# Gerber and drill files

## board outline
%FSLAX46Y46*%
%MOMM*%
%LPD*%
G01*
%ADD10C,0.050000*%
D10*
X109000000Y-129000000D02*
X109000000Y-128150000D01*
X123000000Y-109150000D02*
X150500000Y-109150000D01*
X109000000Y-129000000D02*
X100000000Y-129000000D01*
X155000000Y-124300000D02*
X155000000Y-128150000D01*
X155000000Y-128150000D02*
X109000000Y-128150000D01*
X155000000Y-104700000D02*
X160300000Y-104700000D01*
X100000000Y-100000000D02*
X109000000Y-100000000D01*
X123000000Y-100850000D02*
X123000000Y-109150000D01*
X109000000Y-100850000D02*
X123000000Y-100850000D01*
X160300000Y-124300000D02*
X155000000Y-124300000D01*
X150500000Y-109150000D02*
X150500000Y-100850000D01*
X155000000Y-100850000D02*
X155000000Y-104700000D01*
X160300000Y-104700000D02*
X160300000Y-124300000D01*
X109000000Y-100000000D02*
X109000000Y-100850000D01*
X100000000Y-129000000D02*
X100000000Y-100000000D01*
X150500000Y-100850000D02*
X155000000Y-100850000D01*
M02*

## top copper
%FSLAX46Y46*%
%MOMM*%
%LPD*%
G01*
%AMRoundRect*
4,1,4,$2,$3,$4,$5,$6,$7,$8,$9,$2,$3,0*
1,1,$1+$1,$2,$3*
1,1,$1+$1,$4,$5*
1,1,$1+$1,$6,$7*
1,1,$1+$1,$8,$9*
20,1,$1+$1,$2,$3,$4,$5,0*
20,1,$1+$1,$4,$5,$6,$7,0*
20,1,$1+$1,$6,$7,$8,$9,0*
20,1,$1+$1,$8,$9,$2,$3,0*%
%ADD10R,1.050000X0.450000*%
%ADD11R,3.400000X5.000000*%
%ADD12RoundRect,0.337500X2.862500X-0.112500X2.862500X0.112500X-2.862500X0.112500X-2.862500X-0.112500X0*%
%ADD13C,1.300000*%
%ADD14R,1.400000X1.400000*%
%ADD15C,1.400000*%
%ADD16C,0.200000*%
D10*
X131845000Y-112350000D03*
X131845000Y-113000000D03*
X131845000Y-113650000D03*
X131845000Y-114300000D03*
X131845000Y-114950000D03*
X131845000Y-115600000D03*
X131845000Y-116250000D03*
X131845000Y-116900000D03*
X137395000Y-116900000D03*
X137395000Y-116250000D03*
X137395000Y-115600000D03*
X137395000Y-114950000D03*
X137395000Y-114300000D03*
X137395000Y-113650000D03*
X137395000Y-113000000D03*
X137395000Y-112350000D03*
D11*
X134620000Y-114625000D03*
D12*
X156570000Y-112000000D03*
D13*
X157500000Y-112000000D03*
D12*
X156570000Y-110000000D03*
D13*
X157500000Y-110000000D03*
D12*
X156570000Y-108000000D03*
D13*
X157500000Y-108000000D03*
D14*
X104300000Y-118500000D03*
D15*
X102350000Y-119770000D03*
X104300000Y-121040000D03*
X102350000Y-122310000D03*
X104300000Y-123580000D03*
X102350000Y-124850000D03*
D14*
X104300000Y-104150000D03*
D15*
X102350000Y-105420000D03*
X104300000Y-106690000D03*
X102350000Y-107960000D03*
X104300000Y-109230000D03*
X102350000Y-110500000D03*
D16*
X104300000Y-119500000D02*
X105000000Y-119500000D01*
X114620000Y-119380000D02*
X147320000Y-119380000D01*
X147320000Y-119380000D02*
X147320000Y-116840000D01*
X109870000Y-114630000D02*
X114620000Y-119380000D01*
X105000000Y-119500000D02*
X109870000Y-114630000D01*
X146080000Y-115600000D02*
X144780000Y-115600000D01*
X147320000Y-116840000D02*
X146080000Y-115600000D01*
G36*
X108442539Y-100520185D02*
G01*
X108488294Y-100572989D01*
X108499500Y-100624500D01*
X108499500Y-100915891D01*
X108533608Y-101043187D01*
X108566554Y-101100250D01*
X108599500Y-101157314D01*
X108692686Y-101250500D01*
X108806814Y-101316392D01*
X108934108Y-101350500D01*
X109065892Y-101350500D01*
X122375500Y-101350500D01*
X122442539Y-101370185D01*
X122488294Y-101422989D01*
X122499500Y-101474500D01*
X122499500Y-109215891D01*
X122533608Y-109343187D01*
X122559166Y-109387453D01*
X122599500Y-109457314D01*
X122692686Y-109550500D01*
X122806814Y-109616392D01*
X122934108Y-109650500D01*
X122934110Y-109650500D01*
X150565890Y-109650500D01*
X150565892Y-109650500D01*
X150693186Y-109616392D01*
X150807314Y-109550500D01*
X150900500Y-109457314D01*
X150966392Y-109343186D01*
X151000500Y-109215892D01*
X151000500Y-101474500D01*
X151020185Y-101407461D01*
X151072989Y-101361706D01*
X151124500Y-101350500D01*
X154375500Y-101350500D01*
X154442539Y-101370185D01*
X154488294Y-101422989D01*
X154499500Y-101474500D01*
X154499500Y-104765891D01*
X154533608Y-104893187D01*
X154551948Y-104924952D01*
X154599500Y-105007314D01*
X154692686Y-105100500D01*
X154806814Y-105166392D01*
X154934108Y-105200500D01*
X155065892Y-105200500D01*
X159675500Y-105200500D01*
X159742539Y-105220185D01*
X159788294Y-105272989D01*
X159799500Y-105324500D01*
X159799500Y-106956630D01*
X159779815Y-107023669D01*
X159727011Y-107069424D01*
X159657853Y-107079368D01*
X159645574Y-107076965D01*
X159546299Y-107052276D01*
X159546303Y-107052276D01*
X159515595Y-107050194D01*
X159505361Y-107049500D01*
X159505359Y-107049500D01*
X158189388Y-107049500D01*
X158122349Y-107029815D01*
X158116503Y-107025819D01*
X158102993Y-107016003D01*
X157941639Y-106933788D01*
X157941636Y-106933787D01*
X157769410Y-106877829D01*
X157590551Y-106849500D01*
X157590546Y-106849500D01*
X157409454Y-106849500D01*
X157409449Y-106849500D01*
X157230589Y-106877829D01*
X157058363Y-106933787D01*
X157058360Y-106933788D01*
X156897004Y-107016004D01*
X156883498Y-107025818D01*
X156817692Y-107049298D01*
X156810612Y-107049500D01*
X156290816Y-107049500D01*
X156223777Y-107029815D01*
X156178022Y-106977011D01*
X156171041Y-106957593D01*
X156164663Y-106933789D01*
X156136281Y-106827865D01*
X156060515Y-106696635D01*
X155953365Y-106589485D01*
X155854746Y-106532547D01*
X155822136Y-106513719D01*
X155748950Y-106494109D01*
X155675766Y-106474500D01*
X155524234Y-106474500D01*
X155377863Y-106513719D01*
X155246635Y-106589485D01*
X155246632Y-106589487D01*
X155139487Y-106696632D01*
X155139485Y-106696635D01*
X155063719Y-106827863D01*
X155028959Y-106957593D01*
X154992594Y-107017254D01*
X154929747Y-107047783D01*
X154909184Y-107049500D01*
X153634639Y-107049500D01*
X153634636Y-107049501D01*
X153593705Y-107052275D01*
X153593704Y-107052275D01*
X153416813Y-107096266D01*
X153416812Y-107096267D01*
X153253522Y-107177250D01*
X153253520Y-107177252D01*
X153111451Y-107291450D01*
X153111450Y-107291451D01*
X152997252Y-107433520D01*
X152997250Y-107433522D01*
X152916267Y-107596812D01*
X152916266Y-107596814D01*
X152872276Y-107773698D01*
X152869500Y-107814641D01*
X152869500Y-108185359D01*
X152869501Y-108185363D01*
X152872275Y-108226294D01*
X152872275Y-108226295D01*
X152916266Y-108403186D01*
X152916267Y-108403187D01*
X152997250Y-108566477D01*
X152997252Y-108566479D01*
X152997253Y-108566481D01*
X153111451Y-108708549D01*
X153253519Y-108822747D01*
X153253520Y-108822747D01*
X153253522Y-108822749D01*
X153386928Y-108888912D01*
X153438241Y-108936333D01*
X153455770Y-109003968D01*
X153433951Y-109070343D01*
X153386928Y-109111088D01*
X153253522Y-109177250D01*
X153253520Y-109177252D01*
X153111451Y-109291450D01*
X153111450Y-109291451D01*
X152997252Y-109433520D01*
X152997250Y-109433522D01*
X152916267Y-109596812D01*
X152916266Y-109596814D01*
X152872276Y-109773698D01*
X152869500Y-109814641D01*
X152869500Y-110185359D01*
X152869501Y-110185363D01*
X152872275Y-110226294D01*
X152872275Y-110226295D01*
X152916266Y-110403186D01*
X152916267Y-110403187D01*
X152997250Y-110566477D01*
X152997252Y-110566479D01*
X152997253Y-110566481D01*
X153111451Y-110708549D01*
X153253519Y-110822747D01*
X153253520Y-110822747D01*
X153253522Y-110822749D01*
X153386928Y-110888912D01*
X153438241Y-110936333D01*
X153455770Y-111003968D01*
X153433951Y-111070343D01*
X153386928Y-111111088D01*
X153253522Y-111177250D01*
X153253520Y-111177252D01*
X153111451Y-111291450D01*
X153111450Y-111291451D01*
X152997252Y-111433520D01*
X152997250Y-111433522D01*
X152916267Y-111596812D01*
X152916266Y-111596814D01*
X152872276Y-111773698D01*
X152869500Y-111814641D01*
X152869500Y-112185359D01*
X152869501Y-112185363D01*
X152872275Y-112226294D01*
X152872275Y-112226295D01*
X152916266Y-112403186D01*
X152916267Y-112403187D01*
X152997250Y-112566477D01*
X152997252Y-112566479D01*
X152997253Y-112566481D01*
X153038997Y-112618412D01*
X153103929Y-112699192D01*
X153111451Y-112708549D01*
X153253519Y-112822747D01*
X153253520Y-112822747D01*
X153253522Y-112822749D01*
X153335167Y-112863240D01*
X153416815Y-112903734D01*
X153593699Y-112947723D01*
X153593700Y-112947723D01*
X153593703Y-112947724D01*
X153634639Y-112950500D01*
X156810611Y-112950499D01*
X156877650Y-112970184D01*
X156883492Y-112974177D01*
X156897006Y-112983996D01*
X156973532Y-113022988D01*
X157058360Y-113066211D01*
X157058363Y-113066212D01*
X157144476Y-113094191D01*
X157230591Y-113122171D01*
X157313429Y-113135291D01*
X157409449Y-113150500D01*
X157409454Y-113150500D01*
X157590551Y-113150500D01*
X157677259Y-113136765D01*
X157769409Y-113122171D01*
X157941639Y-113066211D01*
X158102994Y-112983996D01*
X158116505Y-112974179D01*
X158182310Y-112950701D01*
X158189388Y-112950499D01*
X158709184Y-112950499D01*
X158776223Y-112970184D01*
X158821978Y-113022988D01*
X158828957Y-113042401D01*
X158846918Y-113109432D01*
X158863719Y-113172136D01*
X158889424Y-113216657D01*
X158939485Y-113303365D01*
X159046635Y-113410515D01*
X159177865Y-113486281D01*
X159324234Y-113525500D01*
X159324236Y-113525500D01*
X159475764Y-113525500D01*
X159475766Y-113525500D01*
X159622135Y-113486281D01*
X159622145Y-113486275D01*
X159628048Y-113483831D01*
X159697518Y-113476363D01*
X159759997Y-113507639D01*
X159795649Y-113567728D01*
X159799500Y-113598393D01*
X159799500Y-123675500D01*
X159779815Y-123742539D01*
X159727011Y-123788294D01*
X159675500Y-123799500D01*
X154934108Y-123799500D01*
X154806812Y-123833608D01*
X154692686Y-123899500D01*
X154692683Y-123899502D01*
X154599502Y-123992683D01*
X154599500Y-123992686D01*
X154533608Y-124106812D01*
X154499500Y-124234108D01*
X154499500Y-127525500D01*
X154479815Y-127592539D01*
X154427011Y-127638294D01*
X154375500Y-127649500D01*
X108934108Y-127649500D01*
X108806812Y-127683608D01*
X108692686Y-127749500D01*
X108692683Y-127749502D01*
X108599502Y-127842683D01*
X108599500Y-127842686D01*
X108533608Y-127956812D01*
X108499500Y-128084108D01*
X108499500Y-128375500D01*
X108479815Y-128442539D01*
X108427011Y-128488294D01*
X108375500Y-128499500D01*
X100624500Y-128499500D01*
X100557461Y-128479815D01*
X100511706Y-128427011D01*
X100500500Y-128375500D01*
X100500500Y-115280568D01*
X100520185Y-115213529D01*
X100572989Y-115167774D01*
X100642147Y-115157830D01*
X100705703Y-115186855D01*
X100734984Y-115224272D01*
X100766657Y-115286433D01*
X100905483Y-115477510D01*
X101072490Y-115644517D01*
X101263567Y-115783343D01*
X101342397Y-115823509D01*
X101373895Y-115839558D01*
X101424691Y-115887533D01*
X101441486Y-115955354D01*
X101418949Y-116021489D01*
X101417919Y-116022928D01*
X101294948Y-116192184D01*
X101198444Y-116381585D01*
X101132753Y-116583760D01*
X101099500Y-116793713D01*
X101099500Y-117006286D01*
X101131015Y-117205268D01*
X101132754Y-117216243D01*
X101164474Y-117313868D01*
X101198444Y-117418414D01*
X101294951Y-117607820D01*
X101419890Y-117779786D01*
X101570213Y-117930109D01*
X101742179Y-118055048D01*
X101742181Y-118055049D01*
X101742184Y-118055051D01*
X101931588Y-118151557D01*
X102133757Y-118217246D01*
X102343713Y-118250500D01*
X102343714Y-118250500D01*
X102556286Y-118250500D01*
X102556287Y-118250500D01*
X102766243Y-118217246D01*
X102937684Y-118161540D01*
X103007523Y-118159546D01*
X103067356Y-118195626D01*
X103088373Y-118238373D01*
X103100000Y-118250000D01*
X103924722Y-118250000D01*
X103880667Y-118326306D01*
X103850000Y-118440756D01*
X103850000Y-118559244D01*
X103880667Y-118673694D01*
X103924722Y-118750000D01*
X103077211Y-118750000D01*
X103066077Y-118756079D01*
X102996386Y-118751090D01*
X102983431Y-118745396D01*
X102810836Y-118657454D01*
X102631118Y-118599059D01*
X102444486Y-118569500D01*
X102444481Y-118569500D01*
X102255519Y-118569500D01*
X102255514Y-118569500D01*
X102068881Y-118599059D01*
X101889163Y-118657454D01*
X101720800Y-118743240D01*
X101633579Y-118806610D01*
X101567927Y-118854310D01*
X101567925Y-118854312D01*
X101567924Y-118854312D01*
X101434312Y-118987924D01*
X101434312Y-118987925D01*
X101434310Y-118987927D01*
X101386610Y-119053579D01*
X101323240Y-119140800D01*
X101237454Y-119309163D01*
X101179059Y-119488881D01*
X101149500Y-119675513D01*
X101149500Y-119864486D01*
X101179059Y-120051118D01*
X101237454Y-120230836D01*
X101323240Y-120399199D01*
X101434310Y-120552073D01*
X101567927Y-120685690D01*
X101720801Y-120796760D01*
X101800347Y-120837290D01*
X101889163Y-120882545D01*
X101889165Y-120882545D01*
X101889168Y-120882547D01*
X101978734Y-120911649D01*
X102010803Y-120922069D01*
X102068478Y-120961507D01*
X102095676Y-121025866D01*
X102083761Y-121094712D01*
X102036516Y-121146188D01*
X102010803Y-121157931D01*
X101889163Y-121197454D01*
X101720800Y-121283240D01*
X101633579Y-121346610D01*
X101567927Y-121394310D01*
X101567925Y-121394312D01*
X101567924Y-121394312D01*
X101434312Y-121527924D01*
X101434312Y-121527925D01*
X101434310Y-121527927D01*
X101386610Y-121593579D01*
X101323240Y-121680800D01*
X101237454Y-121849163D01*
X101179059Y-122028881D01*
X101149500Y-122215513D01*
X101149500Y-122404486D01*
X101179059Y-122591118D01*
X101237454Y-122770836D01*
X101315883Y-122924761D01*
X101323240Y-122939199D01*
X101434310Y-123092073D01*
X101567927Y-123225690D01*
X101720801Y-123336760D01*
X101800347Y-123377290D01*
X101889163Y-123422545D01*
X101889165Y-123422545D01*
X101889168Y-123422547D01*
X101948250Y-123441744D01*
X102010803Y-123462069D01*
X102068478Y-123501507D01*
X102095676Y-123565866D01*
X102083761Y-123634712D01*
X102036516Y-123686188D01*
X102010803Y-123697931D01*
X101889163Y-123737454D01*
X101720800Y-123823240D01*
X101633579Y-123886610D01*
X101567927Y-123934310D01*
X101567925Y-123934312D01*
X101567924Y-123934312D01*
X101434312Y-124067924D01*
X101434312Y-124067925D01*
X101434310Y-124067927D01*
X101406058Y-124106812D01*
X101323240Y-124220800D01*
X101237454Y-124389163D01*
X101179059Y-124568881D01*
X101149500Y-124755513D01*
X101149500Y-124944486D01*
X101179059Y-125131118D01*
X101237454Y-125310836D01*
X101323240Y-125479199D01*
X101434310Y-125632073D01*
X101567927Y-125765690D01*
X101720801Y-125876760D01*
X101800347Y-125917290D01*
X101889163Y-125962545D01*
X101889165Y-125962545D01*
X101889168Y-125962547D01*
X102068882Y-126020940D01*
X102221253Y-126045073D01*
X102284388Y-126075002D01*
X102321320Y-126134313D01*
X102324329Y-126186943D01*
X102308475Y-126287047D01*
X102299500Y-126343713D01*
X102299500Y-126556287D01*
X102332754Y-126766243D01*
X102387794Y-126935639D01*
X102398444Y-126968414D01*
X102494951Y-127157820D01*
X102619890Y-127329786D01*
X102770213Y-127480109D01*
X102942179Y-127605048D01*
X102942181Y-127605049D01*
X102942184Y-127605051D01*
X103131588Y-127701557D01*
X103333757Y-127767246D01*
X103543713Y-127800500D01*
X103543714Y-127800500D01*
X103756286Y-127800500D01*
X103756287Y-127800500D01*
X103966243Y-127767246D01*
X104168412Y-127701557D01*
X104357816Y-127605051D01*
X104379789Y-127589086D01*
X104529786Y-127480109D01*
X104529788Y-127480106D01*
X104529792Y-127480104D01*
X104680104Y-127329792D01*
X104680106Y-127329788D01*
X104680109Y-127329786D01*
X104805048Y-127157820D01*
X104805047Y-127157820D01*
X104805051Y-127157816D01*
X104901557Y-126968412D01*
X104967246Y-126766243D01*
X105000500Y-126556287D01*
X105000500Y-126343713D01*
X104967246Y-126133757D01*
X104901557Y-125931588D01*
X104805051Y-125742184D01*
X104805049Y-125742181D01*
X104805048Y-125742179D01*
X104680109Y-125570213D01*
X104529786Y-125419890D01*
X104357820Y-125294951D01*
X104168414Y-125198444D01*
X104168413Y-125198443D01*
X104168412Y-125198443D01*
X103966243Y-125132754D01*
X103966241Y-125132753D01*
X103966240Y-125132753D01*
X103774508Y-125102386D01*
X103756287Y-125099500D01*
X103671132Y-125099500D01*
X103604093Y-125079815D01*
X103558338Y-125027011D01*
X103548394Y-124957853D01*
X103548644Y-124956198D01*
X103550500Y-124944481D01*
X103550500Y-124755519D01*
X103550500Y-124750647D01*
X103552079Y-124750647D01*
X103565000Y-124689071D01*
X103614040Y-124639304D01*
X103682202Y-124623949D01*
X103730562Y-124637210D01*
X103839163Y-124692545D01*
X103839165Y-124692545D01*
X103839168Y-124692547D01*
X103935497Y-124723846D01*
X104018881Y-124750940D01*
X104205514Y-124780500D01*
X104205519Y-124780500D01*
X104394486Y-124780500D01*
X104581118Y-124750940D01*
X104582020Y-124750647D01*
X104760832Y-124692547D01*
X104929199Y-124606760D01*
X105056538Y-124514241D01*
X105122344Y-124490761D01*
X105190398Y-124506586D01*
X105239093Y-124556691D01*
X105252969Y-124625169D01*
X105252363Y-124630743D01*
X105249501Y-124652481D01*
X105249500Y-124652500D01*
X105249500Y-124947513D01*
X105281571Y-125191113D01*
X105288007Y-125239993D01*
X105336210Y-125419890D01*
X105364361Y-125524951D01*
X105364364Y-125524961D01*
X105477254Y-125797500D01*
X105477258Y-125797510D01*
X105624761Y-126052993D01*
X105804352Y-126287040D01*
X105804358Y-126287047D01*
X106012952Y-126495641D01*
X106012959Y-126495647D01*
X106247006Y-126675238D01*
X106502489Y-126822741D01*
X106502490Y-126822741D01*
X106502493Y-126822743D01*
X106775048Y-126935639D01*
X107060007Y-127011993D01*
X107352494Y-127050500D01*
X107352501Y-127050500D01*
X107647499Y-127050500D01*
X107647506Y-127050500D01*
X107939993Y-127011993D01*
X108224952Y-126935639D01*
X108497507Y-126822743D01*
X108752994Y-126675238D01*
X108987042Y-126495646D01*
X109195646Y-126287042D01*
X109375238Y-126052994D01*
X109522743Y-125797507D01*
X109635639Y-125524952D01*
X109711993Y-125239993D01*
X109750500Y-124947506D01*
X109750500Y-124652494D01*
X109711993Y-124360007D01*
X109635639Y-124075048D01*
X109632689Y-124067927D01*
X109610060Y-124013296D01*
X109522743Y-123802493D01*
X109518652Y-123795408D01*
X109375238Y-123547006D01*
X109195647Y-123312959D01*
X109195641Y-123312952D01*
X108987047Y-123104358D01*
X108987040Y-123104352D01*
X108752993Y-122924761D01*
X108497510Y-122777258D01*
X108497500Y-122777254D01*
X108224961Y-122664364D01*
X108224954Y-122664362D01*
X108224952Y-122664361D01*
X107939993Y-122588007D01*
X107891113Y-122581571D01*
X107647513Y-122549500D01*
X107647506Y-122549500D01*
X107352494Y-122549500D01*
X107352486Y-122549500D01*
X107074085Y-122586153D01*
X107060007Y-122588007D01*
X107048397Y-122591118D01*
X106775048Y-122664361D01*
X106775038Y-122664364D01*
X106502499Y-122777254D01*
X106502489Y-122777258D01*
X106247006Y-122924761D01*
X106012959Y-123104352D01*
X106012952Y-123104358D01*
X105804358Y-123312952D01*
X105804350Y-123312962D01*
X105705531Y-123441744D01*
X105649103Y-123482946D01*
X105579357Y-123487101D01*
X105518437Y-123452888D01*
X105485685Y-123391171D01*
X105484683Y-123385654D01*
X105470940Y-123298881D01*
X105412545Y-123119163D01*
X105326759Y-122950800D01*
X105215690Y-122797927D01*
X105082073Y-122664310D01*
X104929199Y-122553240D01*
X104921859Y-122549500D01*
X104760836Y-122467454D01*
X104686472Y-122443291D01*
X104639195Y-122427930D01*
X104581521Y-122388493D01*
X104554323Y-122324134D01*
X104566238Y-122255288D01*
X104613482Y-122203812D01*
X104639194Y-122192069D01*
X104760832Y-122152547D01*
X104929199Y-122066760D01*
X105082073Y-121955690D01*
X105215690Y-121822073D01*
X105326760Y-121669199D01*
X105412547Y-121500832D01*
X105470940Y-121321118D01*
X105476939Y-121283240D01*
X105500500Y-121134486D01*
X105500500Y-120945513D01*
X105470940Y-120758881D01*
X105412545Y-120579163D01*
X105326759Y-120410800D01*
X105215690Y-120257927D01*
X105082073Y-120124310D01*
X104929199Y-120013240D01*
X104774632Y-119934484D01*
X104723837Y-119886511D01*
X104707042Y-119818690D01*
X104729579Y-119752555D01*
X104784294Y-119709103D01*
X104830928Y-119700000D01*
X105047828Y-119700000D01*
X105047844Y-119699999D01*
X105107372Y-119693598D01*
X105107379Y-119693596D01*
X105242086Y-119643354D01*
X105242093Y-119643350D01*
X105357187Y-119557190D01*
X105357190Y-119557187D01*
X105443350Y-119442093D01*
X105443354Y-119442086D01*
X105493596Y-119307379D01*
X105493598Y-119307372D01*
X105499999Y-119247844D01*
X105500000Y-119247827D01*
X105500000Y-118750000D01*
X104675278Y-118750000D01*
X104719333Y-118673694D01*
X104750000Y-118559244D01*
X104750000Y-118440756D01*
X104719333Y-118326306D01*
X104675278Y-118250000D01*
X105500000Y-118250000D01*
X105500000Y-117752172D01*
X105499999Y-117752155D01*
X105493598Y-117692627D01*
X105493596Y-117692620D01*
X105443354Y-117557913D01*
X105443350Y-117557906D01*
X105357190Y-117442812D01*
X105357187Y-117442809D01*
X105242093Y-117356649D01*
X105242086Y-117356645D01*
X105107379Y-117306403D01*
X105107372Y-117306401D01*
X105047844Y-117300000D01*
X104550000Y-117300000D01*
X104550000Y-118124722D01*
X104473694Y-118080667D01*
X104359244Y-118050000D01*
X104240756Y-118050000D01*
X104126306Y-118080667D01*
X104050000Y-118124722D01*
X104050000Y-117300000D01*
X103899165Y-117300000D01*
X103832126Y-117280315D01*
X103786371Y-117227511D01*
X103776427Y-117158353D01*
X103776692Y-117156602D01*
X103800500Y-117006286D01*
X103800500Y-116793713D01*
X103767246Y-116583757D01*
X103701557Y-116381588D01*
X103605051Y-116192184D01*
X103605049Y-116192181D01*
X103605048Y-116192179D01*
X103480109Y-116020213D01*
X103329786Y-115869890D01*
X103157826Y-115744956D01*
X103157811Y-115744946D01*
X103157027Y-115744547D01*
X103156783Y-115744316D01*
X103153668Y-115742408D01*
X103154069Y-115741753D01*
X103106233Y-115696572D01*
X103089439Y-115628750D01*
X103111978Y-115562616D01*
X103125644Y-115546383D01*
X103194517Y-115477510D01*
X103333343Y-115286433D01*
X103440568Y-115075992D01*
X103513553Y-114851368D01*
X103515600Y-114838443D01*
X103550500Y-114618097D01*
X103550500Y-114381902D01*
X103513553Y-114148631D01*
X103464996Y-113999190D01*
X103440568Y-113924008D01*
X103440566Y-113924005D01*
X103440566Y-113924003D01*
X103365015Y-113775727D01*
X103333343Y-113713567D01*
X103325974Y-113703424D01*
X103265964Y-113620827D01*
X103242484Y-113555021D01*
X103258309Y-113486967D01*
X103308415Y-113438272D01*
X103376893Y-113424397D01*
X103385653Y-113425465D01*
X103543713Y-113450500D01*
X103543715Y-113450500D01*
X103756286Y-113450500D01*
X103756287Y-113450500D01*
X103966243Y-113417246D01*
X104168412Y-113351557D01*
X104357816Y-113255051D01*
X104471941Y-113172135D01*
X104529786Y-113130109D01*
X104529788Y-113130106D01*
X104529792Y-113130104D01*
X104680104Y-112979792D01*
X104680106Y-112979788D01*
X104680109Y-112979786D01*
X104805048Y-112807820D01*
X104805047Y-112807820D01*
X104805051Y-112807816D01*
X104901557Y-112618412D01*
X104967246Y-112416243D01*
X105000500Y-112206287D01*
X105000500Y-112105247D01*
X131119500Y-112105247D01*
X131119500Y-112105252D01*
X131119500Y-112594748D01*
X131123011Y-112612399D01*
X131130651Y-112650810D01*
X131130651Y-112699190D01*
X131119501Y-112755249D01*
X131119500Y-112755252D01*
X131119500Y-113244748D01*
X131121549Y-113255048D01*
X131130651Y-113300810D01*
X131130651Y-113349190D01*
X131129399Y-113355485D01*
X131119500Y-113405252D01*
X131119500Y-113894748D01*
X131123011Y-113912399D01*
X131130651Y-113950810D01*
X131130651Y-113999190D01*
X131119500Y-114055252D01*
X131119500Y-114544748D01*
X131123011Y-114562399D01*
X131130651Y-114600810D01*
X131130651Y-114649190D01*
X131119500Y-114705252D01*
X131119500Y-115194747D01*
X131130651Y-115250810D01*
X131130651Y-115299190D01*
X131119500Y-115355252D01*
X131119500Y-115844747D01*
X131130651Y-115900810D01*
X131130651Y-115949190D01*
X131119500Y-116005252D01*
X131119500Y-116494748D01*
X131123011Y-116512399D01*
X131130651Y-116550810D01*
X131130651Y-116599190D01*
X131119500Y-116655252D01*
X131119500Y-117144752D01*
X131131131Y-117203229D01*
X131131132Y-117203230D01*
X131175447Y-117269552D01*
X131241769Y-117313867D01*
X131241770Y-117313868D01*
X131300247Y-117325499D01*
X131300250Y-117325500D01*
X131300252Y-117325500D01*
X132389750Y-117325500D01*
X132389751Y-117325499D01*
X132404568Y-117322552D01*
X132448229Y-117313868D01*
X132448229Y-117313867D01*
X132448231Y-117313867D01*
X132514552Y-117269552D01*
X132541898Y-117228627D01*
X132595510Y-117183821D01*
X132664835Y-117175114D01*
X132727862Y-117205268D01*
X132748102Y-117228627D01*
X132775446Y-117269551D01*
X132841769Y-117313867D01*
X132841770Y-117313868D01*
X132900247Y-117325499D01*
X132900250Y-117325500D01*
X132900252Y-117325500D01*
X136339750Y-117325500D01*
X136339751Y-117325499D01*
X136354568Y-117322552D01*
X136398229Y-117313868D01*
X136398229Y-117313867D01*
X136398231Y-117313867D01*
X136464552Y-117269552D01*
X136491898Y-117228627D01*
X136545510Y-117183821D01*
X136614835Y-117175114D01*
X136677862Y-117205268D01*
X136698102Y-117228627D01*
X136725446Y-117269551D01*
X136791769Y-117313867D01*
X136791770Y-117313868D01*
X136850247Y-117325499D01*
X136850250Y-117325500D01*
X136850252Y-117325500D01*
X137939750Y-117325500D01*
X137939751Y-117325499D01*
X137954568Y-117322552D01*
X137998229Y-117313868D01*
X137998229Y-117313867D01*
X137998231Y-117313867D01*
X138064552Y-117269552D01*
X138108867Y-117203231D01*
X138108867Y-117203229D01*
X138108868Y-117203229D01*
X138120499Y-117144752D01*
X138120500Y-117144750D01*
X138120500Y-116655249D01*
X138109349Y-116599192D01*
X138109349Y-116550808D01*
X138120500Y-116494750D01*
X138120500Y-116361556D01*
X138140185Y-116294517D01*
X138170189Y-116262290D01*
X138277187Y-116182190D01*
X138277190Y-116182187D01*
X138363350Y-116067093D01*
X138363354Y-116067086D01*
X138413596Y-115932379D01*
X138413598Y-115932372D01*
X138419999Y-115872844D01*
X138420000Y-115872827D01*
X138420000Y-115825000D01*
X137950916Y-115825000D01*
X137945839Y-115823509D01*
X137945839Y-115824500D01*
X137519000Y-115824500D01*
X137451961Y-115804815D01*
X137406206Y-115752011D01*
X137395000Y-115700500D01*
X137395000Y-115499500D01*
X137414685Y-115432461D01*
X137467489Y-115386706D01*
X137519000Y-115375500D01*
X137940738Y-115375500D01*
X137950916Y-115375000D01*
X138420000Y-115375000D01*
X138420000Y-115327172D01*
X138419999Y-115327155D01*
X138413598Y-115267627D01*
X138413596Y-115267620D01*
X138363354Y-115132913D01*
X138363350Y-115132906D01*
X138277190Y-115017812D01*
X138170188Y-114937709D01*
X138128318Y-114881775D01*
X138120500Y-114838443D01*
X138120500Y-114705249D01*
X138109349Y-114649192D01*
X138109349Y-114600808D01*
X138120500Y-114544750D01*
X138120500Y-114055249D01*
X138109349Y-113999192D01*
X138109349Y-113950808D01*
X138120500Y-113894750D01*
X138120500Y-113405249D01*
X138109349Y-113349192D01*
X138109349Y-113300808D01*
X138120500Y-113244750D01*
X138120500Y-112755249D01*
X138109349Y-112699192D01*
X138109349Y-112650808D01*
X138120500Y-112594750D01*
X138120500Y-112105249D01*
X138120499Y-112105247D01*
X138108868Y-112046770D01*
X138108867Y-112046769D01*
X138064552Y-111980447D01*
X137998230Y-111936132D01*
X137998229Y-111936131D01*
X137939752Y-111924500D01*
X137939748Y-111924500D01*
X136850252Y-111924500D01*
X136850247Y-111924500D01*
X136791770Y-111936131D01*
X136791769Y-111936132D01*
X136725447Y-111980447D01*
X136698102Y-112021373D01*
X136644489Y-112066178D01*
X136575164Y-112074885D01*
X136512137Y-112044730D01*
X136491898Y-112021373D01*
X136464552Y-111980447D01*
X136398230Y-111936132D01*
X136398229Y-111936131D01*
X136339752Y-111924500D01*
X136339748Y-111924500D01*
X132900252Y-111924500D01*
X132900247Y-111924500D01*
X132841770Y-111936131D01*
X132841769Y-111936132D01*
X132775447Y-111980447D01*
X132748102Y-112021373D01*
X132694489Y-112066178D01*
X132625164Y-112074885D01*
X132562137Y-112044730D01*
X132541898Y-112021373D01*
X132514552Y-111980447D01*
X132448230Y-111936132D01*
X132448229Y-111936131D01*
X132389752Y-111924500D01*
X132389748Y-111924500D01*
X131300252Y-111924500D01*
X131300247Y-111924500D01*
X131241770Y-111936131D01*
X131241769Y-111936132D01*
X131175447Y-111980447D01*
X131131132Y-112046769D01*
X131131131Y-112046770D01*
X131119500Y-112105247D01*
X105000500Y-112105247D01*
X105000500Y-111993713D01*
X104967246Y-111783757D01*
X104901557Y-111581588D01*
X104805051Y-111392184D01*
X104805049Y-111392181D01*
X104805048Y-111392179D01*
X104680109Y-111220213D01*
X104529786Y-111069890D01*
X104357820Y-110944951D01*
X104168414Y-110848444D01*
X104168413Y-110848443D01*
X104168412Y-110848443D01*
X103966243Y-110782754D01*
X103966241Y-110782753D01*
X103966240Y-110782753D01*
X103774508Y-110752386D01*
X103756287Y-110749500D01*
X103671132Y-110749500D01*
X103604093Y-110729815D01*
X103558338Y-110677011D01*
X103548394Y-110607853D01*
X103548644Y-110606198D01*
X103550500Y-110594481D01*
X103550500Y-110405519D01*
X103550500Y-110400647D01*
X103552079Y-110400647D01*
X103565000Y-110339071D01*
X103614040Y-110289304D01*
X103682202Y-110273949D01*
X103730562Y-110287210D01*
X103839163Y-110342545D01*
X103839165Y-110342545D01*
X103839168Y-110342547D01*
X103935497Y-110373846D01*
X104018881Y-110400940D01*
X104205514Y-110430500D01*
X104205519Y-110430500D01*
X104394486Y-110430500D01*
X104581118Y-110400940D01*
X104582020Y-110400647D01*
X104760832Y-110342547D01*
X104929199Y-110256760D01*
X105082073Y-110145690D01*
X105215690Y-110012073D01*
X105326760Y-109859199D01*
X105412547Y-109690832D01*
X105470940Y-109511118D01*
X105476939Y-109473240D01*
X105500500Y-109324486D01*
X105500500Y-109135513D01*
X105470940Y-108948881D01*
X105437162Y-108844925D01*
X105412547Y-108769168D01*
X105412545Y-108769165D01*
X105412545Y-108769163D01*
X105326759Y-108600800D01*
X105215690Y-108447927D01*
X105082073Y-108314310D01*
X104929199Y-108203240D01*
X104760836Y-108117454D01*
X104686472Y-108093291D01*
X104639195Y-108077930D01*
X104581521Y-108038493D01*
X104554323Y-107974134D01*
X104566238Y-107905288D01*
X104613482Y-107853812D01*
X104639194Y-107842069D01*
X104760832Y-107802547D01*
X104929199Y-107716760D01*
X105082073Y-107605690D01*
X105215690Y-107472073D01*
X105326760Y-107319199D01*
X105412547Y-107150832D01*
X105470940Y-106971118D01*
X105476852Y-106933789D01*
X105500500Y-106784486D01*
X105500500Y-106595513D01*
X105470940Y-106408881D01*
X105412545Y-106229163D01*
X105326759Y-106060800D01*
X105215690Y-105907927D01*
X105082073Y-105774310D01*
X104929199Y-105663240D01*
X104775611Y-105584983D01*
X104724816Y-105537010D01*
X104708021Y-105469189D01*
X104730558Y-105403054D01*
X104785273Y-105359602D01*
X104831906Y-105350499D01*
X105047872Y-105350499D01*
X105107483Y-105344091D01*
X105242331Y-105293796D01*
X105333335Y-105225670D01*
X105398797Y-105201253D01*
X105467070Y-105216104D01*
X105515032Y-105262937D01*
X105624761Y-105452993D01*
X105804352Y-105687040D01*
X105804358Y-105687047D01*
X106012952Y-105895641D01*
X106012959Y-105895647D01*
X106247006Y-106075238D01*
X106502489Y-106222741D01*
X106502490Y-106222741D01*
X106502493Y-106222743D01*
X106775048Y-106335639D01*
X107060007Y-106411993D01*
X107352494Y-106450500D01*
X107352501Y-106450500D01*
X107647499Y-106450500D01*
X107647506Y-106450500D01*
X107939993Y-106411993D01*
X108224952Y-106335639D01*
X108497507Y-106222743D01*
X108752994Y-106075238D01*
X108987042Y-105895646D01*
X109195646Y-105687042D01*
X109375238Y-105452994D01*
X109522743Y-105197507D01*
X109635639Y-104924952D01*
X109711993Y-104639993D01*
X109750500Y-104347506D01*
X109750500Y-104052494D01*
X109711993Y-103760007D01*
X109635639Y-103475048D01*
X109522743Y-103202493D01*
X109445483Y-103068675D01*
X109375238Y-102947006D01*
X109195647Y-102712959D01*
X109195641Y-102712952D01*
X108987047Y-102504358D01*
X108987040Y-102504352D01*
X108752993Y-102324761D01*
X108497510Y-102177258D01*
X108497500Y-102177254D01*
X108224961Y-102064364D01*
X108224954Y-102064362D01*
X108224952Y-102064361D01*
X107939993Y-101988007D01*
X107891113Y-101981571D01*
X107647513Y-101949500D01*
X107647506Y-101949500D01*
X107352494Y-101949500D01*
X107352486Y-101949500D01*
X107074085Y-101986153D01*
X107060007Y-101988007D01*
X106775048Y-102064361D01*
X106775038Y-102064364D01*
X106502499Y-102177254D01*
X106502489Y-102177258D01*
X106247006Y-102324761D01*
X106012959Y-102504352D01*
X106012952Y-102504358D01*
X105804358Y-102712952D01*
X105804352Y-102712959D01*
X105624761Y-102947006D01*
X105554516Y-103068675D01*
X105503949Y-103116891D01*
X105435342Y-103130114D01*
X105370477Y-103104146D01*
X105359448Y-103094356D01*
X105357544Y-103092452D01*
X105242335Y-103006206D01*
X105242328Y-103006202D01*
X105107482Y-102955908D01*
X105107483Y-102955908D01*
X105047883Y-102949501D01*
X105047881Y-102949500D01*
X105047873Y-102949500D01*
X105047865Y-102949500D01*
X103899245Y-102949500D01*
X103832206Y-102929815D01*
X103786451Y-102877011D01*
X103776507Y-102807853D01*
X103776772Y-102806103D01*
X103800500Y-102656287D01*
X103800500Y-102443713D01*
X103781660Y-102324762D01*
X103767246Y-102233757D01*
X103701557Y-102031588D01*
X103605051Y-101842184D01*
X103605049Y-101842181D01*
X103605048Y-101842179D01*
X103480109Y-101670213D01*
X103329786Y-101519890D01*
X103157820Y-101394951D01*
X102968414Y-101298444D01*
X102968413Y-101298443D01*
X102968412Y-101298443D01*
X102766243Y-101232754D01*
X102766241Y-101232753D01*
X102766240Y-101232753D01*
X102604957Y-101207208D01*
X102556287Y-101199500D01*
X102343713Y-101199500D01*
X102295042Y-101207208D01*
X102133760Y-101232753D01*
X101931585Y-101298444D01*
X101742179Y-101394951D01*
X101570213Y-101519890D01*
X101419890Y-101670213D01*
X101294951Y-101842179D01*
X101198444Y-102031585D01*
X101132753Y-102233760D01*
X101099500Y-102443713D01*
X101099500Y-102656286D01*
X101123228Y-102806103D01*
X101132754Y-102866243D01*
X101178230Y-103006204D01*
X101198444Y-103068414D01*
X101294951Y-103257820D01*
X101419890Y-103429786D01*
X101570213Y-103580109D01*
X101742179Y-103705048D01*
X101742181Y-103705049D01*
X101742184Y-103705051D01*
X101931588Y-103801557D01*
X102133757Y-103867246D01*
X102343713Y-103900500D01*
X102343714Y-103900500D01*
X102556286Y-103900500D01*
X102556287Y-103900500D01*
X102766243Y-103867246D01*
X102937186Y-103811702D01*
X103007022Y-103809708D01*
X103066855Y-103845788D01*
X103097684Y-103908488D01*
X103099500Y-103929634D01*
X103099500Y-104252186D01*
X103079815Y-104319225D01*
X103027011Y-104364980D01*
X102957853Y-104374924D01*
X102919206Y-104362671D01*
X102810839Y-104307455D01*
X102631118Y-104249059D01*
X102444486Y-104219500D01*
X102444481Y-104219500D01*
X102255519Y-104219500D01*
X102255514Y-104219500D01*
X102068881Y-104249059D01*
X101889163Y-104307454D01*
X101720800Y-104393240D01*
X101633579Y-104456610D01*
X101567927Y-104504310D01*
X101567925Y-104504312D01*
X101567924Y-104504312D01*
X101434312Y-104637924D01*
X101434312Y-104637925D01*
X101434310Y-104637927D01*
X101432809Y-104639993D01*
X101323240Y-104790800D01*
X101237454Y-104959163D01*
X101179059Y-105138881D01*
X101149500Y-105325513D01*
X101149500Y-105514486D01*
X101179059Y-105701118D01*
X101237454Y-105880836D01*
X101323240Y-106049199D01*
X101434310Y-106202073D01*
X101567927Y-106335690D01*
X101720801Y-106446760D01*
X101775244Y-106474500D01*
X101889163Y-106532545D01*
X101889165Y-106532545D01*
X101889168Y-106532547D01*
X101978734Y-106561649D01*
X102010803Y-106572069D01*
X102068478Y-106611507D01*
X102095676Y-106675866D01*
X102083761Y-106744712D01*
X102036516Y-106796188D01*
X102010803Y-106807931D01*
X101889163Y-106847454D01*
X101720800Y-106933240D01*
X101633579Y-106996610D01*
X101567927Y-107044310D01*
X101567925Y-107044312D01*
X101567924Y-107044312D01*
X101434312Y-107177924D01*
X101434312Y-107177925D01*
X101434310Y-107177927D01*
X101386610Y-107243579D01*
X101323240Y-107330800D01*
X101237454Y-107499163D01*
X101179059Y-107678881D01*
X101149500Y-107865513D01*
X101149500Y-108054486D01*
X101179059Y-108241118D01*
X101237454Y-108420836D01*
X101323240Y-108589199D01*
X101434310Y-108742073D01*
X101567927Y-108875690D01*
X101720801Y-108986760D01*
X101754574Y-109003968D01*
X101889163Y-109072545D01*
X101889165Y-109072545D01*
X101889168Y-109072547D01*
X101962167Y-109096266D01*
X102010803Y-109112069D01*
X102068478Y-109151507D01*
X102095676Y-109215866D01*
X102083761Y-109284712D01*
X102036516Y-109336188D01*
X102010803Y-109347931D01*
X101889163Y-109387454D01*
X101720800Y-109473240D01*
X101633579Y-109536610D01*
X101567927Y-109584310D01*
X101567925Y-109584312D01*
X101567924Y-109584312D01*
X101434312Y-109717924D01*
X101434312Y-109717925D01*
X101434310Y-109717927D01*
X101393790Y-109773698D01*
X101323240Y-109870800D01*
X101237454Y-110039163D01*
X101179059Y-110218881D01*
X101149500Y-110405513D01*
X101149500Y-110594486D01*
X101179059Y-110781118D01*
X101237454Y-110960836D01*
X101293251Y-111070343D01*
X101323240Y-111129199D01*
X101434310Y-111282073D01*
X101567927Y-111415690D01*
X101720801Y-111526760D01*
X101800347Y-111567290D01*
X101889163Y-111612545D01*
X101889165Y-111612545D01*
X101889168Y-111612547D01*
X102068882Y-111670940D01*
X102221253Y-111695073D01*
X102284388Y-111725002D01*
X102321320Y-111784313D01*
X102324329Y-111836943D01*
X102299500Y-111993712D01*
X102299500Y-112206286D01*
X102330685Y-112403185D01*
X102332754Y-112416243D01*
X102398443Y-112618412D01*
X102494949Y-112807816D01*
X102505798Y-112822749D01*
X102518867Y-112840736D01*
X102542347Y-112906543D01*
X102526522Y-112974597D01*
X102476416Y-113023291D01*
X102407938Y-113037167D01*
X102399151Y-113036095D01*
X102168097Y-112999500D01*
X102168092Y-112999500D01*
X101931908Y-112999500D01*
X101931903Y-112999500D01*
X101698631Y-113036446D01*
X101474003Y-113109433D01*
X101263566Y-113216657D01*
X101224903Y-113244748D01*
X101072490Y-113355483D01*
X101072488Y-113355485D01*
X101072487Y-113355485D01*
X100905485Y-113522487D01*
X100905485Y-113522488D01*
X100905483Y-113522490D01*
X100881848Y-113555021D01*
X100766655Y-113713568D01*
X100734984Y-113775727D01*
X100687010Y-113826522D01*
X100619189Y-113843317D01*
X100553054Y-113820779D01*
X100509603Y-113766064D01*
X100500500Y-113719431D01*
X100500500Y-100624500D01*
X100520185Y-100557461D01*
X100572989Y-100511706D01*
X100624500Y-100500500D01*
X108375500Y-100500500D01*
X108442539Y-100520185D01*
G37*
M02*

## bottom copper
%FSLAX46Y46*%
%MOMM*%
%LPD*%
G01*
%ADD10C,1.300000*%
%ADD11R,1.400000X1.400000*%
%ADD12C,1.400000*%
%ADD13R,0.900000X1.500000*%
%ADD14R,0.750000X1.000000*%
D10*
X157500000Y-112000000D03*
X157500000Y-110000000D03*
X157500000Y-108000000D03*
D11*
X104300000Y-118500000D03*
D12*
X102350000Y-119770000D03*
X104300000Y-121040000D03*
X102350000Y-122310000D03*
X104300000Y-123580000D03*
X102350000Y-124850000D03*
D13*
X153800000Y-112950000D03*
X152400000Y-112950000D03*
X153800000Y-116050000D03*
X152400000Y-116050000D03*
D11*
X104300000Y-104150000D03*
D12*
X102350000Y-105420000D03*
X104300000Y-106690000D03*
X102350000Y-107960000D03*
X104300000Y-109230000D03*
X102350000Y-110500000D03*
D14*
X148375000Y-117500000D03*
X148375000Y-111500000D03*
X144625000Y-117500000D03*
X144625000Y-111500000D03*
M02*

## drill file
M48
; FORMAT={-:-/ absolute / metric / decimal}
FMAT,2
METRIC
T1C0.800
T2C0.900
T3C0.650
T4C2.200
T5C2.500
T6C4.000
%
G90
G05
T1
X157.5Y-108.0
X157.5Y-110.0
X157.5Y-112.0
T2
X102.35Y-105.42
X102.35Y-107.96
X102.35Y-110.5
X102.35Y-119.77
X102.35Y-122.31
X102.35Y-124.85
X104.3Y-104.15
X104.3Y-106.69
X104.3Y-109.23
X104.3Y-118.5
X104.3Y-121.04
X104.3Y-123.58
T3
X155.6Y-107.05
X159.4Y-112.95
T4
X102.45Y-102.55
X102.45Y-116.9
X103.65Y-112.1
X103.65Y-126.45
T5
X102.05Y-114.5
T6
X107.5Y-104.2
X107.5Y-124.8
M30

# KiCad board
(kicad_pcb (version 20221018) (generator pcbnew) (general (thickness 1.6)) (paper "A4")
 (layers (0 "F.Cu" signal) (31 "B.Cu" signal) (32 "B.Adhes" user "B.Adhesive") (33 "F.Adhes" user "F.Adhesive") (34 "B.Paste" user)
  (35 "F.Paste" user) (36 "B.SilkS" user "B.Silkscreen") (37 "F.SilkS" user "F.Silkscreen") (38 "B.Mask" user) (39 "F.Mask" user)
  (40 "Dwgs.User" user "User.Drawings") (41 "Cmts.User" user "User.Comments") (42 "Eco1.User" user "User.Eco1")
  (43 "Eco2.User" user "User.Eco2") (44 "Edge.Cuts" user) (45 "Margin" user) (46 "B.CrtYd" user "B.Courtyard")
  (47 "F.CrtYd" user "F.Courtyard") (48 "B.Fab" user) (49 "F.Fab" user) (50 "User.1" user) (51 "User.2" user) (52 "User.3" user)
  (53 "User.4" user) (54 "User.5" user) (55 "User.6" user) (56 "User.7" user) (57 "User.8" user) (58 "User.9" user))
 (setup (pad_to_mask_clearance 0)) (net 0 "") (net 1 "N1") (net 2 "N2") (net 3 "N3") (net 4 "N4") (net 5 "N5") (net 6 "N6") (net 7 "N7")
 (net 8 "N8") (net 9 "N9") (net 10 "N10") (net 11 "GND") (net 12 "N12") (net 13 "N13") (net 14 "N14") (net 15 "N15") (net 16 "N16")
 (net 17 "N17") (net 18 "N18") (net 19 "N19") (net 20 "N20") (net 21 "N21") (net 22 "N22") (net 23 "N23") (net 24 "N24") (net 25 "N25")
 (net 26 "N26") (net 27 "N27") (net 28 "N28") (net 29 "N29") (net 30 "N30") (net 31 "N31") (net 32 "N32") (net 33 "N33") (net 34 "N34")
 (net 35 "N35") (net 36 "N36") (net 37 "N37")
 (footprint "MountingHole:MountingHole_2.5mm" (layer "F.Cu") (at 102.05 114.5)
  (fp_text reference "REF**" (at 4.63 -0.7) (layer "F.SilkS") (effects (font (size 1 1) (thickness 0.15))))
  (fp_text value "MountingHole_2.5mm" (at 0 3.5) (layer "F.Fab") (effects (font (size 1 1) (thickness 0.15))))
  (pad "" np_thru_hole circle (at 0 0) (size 2.5 2.5) (drill 2.5) (layers "*.Cu" "*.Mask")))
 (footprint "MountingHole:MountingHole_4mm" (layer "F.Cu") (at 107.5 104.2)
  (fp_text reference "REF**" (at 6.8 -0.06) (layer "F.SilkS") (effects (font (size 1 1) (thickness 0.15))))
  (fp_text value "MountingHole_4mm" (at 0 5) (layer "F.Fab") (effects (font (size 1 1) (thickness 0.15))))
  (pad "" np_thru_hole circle (at 0 0) (size 4 4) (drill 4) (layers "*.Cu" "*.Mask")))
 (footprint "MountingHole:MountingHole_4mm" (layer "F.Cu") (at 107.5 124.8)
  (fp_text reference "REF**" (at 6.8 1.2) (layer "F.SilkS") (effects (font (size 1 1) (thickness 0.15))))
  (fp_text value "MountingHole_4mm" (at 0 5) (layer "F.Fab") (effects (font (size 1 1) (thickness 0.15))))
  (pad "" np_thru_hole circle (at 0 0) (size 4 4) (drill 4) (layers "*.Cu" "*.Mask")))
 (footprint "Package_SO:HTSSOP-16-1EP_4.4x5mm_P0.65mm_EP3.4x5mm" (layer "F.Cu") (at 134.62 114.625) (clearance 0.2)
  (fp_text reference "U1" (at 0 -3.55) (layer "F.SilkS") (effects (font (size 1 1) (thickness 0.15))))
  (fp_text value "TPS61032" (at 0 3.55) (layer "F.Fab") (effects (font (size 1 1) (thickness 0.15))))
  (pad "" smd rect (at -1.1334 -1.875) (size 0.88 1.05) (layers "F.Paste"))
  (pad "" smd rect (at -1.1334 -0.625) (size 0.88 1.05) (layers "F.Paste"))
  (pad "" smd rect (at -1.1334 0.625) (size 0.88 1.05) (layers "F.Paste"))
  (pad "" smd rect (at -1.1334 1.875) (size 0.88 1.05) (layers "F.Paste"))
  (pad "" smd rect (at 0 -1.875) (size 0.88 1.05) (layers "F.Paste"))
  (pad "" smd rect (at 0 -0.625) (size 0.88 1.05) (layers "F.Paste"))
  (pad "" smd rect (at 0 0.625) (size 0.88 1.05) (layers "F.Paste"))
  (pad "" smd rect (at 0 1.875) (size 0.88 1.05) (layers "F.Paste"))
  (pad "" smd rect (at 1.1334 -1.875) (size 0.88 1.05) (layers "F.Paste"))
  (pad "" smd rect (at 1.1334 -0.625) (size 0.88 1.05) (layers "F.Paste"))
  (pad "" smd rect (at 1.1334 0.625) (size 0.88 1.05) (layers "F.Paste"))
  (pad "" smd rect (at 1.1334 1.875) (size 0.88 1.05) (layers "F.Paste"))
  (pad "1" smd rect (at -2.775 -2.275) (size 1.05 0.45) (layers "F.Cu" "F.Paste" "F.Mask") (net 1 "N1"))
  (pad "2" smd rect (at -2.775 -1.625) (size 1.05 0.45) (layers "F.Cu" "F.Paste" "F.Mask") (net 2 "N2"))
  (pad "3" smd rect (at -2.775 -0.975) (size 1.05 0.45) (layers "F.Cu" "F.Paste" "F.Mask") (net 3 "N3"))
  (pad "4" smd rect (at -2.775 -0.325) (size 1.05 0.45) (layers "F.Cu" "F.Paste" "F.Mask") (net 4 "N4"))
  (pad "5" smd rect (at -2.775 0.325) (size 1.05 0.45) (layers "F.Cu" "F.Paste" "F.Mask") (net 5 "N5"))
  (pad "6" smd rect (at -2.775 0.975) (size 1.05 0.45) (layers "F.Cu" "F.Paste" "F.Mask") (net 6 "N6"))
  (pad "7" smd rect (at -2.775 1.625) (size 1.05 0.45) (layers "F.Cu" "F.Paste" "F.Mask") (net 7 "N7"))
  (pad "8" smd rect (at -2.775 2.275) (size 1.05 0.45) (layers "F.Cu" "F.Paste" "F.Mask") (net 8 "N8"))
  (pad "9" smd rect (at 2.775 2.275) (size 1.05 0.45) (layers "F.Cu" "F.Paste" "F.Mask") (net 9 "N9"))
  (pad "10" smd rect (at 2.775 1.625) (size 1.05 0.45) (layers "F.Cu" "F.Paste" "F.Mask") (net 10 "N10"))
  (pad "11" smd rect (at 2.775 0.975) (size 1.05 0.45) (layers "F.Cu" "F.Paste" "F.Mask") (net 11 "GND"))
  (pad "12" smd rect (at 2.775 0.325) (size 1.05 0.45) (layers "F.Cu" "F.Paste" "F.Mask") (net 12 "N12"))
  (pad "13" smd rect (at 2.775 -0.325) (size 1.05 0.45) (layers "F.Cu" "F.Paste" "F.Mask") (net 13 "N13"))
  (pad "14" smd rect (at 2.775 -0.975) (size 1.05 0.45) (layers "F.Cu" "F.Paste" "F.Mask") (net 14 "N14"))
  (pad "15" smd rect (at 2.775 -1.625) (size 1.05 0.45) (layers "F.Cu" "F.Paste" "F.Mask") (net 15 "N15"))
  (pad "16" smd rect (at 2.775 -2.275) (size 1.05 0.45) (layers "F.Cu" "F.Paste" "F.Mask") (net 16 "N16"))
  (pad "17" smd rect (at 0 0) (size 3.4 5) (layers "F.Cu" "F.Mask") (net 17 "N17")))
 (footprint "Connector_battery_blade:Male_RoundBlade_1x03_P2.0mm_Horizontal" (layer "F.Cu") (at 157.5 110 90)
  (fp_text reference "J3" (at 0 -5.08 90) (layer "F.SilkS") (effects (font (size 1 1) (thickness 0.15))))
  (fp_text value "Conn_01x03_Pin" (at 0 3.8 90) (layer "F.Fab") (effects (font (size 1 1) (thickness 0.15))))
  (pad "" np_thru_hole circle (at -2.95 1.9 90) (size 0.65 0.65) (drill 0.65) (layers "F&B.Cu" "*.Mask"))
  (pad "" np_thru_hole circle (at 2.95 -1.9 90) (size 0.65 0.65) (drill 0.65) (layers "F&B.Cu" "*.Mask"))
  (pad "1" smd roundrect (at -2 -0.93 90) (size 0.9 6.4) (layers "F.Cu" "F.Paste" "F.Mask") (roundrect_rratio 0.375) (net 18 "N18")
   (thermal_bridge_angle 45))
  (pad "1" thru_hole circle (at -2 0 90) (size 1.3 1.3) (drill 0.8) (layers "*.Cu" "*.Mask") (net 18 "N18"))
  (pad "2" smd roundrect (at 0 -0.93 90) (size 0.9 6.4) (layers "F.Cu" "F.Paste" "F.Mask") (roundrect_rratio 0.375) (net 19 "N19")
   (thermal_bridge_angle 45))
  (pad "2" thru_hole circle (at 0 0 90) (size 1.3 1.3) (drill 0.8) (layers "*.Cu" "*.Mask") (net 19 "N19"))
  (pad "3" smd roundrect (at 2 -0.93 90) (size 0.9 6.4) (layers "F.Cu" "F.Paste" "F.Mask") (roundrect_rratio 0.375) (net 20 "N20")
   (thermal_bridge_angle 45))
  (pad "3" thru_hole circle (at 2 0 90) (size 1.3 1.3) (drill 0.8) (layers "*.Cu" "*.Mask") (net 20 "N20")))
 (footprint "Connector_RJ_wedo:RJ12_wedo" (layer "B.Cu") (at 104.3 118.5 -90)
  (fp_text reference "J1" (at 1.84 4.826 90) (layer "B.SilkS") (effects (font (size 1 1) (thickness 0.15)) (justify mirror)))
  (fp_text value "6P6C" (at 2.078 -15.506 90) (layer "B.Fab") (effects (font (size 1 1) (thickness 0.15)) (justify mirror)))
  (pad "" np_thru_hole circle (at -1.6 1.85 270) (size 2.25 2.25) (drill 2.2) (layers "*.Mask"))
  (pad "" np_thru_hole circle (at 7.95 0.65 270) (size 2.25 2.25) (drill 2.2) (layers "*.Mask"))
  (pad "1" thru_hole rect (at 0 0 270) (size 1.4 1.4) (drill 0.9) (layers "*.Cu" "*.Mask") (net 11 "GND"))
  (pad "2" thru_hole circle (at 1.27 1.95 270) (size 1.4 1.4) (drill 0.9) (layers "*.Cu" "*.Mask") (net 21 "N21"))
  (pad "3" thru_hole circle (at 2.54 0 270) (size 1.4 1.4) (drill 0.9) (layers "*.Cu" "*.Mask") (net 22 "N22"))
  (pad "4" thru_hole circle (at 3.81 1.95 270) (size 1.4 1.4) (drill 0.9) (layers "*.Cu" "*.Mask") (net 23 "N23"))
  (pad "5" thru_hole circle (at 5.08 0 270) (size 1.4 1.4) (drill 0.9) (layers "*.Cu" "*.Mask") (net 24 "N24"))
  (pad "6" thru_hole circle (at 6.35 1.95 270) (size 1.4 1.4) (drill 0.9) (layers "*.Cu" "*.Mask") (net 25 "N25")))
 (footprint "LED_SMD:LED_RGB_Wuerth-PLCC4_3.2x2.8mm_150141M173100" (layer "B.Cu") (at 153.1 114.5 90)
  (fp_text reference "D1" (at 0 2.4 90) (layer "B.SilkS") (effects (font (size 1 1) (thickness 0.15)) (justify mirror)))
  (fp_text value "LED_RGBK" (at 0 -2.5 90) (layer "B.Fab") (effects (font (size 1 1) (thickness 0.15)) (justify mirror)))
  (pad "1" smd rect (at 1.55 0.7 90) (size 1.5 0.9) (layers "B.Cu" "B.Paste" "B.Mask") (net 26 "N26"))
  (pad "2" smd rect (at 1.55 -0.7 90) (size 1.5 0.9) (layers "B.Cu" "B.Paste" "B.Mask") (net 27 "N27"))
  (pad "3" smd rect (at -1.55 0.7 90) (size 1.5 0.9) (layers "B.Cu" "B.Paste" "B.Mask") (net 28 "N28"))
  (pad "4" smd rect (at -1.55 -0.7 90) (size 1.5 0.9) (layers "B.Cu" "B.Paste" "B.Mask") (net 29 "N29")))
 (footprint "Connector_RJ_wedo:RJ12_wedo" (layer "B.Cu") (at 104.3 104.15 -90)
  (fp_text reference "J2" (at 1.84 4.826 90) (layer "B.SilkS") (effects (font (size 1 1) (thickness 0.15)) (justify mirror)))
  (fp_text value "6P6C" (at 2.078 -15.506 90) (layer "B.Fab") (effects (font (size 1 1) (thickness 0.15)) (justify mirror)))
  (pad "" np_thru_hole circle (at -1.6 1.85 270) (size 2.25 2.25) (drill 2.2) (layers "*.Mask"))
  (pad "" np_thru_hole circle (at 7.95 0.65 270) (size 2.25 2.25) (drill 2.2) (layers "*.Mask"))
  (pad "1" thru_hole rect (at 0 0 270) (size 1.4 1.4) (drill 0.9) (layers "*.Cu" "*.Mask") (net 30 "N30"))
  (pad "2" thru_hole circle (at 1.27 1.95 270) (size 1.4 1.4) (drill 0.9) (layers "*.Cu" "*.Mask") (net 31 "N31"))
  (pad "3" thru_hole circle (at 2.54 0 270) (size 1.4 1.4) (drill 0.9) (layers "*.Cu" "*.Mask") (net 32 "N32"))
  (pad "4" thru_hole circle (at 3.81 1.95 270) (size 1.4 1.4) (drill 0.9) (layers "*.Cu" "*.Mask") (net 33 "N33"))
  (pad "5" thru_hole circle (at 5.08 0 270) (size 1.4 1.4) (drill 0.9) (layers "*.Cu" "*.Mask") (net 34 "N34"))
  (pad "6" thru_hole circle (at 6.35 1.95 270) (size 1.4 1.4) (drill 0.9) (layers "*.Cu" "*.Mask") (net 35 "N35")))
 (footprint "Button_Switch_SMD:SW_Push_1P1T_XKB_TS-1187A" (layer "B.Cu") (at 146.5 114.5 90)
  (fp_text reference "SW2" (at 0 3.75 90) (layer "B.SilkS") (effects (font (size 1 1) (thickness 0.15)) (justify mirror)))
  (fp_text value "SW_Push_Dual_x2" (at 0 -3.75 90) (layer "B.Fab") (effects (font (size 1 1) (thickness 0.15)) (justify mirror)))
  (pad "1" smd rect (at -3 1.875 90) (size 1 0.75) (layers "B.Cu" "B.Paste" "B.Mask") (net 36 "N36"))
  (pad "1" smd rect (at 3 1.875 90) (size 1 0.75) (layers "B.Cu" "B.Paste" "B.Mask") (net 36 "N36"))
  (pad "2" smd rect (at -3 -1.875 90) (size 1 0.75) (layers "B.Cu" "B.Paste" "B.Mask") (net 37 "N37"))
  (pad "2" smd rect (at 3 -1.875 90) (size 1 0.75) (layers "B.Cu" "B.Paste" "B.Mask") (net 37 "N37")))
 (gr_line (start 109 129) (end 109 128.15) (stroke (width 0.05) (type default)) (layer "Edge.Cuts"))
 (gr_line (start 123 109.15) (end 150.5 109.15) (stroke (width 0.05) (type default)) (layer "Edge.Cuts"))
 (gr_line (start 109 129) (end 100 129) (stroke (width 0.05) (type default)) (layer "Edge.Cuts"))
 (gr_line (start 155 124.3) (end 155 128.15) (stroke (width 0.05) (type default)) (layer "Edge.Cuts"))
 (gr_line (start 155 128.15) (end 109 128.15) (stroke (width 0.05) (type default)) (layer "Edge.Cuts"))
 (gr_line (start 155 104.7) (end 160.3 104.7) (stroke (width 0.05) (type default)) (layer "Edge.Cuts"))
 (gr_line (start 100 100) (end 109 100) (stroke (width 0.05) (type default)) (layer "Edge.Cuts"))
 (gr_line (start 123 100.85) (end 123 109.15) (stroke (width 0.05) (type default)) (layer "Edge.Cuts"))
 (gr_line (start 109 100.85) (end 123 100.85) (stroke (width 0.05) (type default)) (layer "Edge.Cuts"))
 (gr_line (start 160.3 124.3) (end 155 124.3) (stroke (width 0.05) (type default)) (layer "Edge.Cuts"))
 (gr_line (start 150.5 109.15) (end 150.5 100.85) (stroke (width 0.05) (type default)) (layer "Edge.Cuts"))
 (gr_line (start 155 100.85) (end 155 104.7) (stroke (width 0.05) (type default)) (layer "Edge.Cuts"))
 (gr_line (start 160.3 104.7) (end 160.3 124.3) (stroke (width 0.05) (type default)) (layer "Edge.Cuts"))
 (gr_line (start 109 100) (end 109 100.85) (stroke (width 0.05) (type default)) (layer "Edge.Cuts"))
 (gr_line (start 100 129) (end 100 100) (stroke (width 0.05) (type default)) (layer "Edge.Cuts"))
 (gr_line (start 150.5 100.85) (end 155 100.85) (stroke (width 0.05) (type default)) (layer "Edge.Cuts"))
 (segment (start 104.3 119.5) (end 105 119.5) (width 0.2) (layer "F.Cu") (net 11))
 (segment (start 114.62 119.38) (end 147.32 119.38) (width 0.2) (layer "F.Cu") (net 11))
 (segment (start 147.32 119.38) (end 147.32 116.84) (width 0.2) (layer "F.Cu") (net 11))
 (segment (start 109.87 114.63) (end 114.62 119.38) (width 0.2) (layer "F.Cu") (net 11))
 (segment (start 105 119.5) (end 109.87 114.63) (width 0.2) (layer "F.Cu") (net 11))
 (segment (start 146.08 115.6) (end 144.78 115.6) (width 0.2) (layer "F.Cu") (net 11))
 (segment (start 147.32 116.84) (end 146.08 115.6) (width 0.2) (layer "F.Cu") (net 11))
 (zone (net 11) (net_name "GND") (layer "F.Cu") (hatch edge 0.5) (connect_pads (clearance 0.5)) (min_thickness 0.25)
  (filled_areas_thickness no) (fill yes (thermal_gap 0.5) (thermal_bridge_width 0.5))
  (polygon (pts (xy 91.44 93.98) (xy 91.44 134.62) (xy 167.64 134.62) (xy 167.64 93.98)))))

